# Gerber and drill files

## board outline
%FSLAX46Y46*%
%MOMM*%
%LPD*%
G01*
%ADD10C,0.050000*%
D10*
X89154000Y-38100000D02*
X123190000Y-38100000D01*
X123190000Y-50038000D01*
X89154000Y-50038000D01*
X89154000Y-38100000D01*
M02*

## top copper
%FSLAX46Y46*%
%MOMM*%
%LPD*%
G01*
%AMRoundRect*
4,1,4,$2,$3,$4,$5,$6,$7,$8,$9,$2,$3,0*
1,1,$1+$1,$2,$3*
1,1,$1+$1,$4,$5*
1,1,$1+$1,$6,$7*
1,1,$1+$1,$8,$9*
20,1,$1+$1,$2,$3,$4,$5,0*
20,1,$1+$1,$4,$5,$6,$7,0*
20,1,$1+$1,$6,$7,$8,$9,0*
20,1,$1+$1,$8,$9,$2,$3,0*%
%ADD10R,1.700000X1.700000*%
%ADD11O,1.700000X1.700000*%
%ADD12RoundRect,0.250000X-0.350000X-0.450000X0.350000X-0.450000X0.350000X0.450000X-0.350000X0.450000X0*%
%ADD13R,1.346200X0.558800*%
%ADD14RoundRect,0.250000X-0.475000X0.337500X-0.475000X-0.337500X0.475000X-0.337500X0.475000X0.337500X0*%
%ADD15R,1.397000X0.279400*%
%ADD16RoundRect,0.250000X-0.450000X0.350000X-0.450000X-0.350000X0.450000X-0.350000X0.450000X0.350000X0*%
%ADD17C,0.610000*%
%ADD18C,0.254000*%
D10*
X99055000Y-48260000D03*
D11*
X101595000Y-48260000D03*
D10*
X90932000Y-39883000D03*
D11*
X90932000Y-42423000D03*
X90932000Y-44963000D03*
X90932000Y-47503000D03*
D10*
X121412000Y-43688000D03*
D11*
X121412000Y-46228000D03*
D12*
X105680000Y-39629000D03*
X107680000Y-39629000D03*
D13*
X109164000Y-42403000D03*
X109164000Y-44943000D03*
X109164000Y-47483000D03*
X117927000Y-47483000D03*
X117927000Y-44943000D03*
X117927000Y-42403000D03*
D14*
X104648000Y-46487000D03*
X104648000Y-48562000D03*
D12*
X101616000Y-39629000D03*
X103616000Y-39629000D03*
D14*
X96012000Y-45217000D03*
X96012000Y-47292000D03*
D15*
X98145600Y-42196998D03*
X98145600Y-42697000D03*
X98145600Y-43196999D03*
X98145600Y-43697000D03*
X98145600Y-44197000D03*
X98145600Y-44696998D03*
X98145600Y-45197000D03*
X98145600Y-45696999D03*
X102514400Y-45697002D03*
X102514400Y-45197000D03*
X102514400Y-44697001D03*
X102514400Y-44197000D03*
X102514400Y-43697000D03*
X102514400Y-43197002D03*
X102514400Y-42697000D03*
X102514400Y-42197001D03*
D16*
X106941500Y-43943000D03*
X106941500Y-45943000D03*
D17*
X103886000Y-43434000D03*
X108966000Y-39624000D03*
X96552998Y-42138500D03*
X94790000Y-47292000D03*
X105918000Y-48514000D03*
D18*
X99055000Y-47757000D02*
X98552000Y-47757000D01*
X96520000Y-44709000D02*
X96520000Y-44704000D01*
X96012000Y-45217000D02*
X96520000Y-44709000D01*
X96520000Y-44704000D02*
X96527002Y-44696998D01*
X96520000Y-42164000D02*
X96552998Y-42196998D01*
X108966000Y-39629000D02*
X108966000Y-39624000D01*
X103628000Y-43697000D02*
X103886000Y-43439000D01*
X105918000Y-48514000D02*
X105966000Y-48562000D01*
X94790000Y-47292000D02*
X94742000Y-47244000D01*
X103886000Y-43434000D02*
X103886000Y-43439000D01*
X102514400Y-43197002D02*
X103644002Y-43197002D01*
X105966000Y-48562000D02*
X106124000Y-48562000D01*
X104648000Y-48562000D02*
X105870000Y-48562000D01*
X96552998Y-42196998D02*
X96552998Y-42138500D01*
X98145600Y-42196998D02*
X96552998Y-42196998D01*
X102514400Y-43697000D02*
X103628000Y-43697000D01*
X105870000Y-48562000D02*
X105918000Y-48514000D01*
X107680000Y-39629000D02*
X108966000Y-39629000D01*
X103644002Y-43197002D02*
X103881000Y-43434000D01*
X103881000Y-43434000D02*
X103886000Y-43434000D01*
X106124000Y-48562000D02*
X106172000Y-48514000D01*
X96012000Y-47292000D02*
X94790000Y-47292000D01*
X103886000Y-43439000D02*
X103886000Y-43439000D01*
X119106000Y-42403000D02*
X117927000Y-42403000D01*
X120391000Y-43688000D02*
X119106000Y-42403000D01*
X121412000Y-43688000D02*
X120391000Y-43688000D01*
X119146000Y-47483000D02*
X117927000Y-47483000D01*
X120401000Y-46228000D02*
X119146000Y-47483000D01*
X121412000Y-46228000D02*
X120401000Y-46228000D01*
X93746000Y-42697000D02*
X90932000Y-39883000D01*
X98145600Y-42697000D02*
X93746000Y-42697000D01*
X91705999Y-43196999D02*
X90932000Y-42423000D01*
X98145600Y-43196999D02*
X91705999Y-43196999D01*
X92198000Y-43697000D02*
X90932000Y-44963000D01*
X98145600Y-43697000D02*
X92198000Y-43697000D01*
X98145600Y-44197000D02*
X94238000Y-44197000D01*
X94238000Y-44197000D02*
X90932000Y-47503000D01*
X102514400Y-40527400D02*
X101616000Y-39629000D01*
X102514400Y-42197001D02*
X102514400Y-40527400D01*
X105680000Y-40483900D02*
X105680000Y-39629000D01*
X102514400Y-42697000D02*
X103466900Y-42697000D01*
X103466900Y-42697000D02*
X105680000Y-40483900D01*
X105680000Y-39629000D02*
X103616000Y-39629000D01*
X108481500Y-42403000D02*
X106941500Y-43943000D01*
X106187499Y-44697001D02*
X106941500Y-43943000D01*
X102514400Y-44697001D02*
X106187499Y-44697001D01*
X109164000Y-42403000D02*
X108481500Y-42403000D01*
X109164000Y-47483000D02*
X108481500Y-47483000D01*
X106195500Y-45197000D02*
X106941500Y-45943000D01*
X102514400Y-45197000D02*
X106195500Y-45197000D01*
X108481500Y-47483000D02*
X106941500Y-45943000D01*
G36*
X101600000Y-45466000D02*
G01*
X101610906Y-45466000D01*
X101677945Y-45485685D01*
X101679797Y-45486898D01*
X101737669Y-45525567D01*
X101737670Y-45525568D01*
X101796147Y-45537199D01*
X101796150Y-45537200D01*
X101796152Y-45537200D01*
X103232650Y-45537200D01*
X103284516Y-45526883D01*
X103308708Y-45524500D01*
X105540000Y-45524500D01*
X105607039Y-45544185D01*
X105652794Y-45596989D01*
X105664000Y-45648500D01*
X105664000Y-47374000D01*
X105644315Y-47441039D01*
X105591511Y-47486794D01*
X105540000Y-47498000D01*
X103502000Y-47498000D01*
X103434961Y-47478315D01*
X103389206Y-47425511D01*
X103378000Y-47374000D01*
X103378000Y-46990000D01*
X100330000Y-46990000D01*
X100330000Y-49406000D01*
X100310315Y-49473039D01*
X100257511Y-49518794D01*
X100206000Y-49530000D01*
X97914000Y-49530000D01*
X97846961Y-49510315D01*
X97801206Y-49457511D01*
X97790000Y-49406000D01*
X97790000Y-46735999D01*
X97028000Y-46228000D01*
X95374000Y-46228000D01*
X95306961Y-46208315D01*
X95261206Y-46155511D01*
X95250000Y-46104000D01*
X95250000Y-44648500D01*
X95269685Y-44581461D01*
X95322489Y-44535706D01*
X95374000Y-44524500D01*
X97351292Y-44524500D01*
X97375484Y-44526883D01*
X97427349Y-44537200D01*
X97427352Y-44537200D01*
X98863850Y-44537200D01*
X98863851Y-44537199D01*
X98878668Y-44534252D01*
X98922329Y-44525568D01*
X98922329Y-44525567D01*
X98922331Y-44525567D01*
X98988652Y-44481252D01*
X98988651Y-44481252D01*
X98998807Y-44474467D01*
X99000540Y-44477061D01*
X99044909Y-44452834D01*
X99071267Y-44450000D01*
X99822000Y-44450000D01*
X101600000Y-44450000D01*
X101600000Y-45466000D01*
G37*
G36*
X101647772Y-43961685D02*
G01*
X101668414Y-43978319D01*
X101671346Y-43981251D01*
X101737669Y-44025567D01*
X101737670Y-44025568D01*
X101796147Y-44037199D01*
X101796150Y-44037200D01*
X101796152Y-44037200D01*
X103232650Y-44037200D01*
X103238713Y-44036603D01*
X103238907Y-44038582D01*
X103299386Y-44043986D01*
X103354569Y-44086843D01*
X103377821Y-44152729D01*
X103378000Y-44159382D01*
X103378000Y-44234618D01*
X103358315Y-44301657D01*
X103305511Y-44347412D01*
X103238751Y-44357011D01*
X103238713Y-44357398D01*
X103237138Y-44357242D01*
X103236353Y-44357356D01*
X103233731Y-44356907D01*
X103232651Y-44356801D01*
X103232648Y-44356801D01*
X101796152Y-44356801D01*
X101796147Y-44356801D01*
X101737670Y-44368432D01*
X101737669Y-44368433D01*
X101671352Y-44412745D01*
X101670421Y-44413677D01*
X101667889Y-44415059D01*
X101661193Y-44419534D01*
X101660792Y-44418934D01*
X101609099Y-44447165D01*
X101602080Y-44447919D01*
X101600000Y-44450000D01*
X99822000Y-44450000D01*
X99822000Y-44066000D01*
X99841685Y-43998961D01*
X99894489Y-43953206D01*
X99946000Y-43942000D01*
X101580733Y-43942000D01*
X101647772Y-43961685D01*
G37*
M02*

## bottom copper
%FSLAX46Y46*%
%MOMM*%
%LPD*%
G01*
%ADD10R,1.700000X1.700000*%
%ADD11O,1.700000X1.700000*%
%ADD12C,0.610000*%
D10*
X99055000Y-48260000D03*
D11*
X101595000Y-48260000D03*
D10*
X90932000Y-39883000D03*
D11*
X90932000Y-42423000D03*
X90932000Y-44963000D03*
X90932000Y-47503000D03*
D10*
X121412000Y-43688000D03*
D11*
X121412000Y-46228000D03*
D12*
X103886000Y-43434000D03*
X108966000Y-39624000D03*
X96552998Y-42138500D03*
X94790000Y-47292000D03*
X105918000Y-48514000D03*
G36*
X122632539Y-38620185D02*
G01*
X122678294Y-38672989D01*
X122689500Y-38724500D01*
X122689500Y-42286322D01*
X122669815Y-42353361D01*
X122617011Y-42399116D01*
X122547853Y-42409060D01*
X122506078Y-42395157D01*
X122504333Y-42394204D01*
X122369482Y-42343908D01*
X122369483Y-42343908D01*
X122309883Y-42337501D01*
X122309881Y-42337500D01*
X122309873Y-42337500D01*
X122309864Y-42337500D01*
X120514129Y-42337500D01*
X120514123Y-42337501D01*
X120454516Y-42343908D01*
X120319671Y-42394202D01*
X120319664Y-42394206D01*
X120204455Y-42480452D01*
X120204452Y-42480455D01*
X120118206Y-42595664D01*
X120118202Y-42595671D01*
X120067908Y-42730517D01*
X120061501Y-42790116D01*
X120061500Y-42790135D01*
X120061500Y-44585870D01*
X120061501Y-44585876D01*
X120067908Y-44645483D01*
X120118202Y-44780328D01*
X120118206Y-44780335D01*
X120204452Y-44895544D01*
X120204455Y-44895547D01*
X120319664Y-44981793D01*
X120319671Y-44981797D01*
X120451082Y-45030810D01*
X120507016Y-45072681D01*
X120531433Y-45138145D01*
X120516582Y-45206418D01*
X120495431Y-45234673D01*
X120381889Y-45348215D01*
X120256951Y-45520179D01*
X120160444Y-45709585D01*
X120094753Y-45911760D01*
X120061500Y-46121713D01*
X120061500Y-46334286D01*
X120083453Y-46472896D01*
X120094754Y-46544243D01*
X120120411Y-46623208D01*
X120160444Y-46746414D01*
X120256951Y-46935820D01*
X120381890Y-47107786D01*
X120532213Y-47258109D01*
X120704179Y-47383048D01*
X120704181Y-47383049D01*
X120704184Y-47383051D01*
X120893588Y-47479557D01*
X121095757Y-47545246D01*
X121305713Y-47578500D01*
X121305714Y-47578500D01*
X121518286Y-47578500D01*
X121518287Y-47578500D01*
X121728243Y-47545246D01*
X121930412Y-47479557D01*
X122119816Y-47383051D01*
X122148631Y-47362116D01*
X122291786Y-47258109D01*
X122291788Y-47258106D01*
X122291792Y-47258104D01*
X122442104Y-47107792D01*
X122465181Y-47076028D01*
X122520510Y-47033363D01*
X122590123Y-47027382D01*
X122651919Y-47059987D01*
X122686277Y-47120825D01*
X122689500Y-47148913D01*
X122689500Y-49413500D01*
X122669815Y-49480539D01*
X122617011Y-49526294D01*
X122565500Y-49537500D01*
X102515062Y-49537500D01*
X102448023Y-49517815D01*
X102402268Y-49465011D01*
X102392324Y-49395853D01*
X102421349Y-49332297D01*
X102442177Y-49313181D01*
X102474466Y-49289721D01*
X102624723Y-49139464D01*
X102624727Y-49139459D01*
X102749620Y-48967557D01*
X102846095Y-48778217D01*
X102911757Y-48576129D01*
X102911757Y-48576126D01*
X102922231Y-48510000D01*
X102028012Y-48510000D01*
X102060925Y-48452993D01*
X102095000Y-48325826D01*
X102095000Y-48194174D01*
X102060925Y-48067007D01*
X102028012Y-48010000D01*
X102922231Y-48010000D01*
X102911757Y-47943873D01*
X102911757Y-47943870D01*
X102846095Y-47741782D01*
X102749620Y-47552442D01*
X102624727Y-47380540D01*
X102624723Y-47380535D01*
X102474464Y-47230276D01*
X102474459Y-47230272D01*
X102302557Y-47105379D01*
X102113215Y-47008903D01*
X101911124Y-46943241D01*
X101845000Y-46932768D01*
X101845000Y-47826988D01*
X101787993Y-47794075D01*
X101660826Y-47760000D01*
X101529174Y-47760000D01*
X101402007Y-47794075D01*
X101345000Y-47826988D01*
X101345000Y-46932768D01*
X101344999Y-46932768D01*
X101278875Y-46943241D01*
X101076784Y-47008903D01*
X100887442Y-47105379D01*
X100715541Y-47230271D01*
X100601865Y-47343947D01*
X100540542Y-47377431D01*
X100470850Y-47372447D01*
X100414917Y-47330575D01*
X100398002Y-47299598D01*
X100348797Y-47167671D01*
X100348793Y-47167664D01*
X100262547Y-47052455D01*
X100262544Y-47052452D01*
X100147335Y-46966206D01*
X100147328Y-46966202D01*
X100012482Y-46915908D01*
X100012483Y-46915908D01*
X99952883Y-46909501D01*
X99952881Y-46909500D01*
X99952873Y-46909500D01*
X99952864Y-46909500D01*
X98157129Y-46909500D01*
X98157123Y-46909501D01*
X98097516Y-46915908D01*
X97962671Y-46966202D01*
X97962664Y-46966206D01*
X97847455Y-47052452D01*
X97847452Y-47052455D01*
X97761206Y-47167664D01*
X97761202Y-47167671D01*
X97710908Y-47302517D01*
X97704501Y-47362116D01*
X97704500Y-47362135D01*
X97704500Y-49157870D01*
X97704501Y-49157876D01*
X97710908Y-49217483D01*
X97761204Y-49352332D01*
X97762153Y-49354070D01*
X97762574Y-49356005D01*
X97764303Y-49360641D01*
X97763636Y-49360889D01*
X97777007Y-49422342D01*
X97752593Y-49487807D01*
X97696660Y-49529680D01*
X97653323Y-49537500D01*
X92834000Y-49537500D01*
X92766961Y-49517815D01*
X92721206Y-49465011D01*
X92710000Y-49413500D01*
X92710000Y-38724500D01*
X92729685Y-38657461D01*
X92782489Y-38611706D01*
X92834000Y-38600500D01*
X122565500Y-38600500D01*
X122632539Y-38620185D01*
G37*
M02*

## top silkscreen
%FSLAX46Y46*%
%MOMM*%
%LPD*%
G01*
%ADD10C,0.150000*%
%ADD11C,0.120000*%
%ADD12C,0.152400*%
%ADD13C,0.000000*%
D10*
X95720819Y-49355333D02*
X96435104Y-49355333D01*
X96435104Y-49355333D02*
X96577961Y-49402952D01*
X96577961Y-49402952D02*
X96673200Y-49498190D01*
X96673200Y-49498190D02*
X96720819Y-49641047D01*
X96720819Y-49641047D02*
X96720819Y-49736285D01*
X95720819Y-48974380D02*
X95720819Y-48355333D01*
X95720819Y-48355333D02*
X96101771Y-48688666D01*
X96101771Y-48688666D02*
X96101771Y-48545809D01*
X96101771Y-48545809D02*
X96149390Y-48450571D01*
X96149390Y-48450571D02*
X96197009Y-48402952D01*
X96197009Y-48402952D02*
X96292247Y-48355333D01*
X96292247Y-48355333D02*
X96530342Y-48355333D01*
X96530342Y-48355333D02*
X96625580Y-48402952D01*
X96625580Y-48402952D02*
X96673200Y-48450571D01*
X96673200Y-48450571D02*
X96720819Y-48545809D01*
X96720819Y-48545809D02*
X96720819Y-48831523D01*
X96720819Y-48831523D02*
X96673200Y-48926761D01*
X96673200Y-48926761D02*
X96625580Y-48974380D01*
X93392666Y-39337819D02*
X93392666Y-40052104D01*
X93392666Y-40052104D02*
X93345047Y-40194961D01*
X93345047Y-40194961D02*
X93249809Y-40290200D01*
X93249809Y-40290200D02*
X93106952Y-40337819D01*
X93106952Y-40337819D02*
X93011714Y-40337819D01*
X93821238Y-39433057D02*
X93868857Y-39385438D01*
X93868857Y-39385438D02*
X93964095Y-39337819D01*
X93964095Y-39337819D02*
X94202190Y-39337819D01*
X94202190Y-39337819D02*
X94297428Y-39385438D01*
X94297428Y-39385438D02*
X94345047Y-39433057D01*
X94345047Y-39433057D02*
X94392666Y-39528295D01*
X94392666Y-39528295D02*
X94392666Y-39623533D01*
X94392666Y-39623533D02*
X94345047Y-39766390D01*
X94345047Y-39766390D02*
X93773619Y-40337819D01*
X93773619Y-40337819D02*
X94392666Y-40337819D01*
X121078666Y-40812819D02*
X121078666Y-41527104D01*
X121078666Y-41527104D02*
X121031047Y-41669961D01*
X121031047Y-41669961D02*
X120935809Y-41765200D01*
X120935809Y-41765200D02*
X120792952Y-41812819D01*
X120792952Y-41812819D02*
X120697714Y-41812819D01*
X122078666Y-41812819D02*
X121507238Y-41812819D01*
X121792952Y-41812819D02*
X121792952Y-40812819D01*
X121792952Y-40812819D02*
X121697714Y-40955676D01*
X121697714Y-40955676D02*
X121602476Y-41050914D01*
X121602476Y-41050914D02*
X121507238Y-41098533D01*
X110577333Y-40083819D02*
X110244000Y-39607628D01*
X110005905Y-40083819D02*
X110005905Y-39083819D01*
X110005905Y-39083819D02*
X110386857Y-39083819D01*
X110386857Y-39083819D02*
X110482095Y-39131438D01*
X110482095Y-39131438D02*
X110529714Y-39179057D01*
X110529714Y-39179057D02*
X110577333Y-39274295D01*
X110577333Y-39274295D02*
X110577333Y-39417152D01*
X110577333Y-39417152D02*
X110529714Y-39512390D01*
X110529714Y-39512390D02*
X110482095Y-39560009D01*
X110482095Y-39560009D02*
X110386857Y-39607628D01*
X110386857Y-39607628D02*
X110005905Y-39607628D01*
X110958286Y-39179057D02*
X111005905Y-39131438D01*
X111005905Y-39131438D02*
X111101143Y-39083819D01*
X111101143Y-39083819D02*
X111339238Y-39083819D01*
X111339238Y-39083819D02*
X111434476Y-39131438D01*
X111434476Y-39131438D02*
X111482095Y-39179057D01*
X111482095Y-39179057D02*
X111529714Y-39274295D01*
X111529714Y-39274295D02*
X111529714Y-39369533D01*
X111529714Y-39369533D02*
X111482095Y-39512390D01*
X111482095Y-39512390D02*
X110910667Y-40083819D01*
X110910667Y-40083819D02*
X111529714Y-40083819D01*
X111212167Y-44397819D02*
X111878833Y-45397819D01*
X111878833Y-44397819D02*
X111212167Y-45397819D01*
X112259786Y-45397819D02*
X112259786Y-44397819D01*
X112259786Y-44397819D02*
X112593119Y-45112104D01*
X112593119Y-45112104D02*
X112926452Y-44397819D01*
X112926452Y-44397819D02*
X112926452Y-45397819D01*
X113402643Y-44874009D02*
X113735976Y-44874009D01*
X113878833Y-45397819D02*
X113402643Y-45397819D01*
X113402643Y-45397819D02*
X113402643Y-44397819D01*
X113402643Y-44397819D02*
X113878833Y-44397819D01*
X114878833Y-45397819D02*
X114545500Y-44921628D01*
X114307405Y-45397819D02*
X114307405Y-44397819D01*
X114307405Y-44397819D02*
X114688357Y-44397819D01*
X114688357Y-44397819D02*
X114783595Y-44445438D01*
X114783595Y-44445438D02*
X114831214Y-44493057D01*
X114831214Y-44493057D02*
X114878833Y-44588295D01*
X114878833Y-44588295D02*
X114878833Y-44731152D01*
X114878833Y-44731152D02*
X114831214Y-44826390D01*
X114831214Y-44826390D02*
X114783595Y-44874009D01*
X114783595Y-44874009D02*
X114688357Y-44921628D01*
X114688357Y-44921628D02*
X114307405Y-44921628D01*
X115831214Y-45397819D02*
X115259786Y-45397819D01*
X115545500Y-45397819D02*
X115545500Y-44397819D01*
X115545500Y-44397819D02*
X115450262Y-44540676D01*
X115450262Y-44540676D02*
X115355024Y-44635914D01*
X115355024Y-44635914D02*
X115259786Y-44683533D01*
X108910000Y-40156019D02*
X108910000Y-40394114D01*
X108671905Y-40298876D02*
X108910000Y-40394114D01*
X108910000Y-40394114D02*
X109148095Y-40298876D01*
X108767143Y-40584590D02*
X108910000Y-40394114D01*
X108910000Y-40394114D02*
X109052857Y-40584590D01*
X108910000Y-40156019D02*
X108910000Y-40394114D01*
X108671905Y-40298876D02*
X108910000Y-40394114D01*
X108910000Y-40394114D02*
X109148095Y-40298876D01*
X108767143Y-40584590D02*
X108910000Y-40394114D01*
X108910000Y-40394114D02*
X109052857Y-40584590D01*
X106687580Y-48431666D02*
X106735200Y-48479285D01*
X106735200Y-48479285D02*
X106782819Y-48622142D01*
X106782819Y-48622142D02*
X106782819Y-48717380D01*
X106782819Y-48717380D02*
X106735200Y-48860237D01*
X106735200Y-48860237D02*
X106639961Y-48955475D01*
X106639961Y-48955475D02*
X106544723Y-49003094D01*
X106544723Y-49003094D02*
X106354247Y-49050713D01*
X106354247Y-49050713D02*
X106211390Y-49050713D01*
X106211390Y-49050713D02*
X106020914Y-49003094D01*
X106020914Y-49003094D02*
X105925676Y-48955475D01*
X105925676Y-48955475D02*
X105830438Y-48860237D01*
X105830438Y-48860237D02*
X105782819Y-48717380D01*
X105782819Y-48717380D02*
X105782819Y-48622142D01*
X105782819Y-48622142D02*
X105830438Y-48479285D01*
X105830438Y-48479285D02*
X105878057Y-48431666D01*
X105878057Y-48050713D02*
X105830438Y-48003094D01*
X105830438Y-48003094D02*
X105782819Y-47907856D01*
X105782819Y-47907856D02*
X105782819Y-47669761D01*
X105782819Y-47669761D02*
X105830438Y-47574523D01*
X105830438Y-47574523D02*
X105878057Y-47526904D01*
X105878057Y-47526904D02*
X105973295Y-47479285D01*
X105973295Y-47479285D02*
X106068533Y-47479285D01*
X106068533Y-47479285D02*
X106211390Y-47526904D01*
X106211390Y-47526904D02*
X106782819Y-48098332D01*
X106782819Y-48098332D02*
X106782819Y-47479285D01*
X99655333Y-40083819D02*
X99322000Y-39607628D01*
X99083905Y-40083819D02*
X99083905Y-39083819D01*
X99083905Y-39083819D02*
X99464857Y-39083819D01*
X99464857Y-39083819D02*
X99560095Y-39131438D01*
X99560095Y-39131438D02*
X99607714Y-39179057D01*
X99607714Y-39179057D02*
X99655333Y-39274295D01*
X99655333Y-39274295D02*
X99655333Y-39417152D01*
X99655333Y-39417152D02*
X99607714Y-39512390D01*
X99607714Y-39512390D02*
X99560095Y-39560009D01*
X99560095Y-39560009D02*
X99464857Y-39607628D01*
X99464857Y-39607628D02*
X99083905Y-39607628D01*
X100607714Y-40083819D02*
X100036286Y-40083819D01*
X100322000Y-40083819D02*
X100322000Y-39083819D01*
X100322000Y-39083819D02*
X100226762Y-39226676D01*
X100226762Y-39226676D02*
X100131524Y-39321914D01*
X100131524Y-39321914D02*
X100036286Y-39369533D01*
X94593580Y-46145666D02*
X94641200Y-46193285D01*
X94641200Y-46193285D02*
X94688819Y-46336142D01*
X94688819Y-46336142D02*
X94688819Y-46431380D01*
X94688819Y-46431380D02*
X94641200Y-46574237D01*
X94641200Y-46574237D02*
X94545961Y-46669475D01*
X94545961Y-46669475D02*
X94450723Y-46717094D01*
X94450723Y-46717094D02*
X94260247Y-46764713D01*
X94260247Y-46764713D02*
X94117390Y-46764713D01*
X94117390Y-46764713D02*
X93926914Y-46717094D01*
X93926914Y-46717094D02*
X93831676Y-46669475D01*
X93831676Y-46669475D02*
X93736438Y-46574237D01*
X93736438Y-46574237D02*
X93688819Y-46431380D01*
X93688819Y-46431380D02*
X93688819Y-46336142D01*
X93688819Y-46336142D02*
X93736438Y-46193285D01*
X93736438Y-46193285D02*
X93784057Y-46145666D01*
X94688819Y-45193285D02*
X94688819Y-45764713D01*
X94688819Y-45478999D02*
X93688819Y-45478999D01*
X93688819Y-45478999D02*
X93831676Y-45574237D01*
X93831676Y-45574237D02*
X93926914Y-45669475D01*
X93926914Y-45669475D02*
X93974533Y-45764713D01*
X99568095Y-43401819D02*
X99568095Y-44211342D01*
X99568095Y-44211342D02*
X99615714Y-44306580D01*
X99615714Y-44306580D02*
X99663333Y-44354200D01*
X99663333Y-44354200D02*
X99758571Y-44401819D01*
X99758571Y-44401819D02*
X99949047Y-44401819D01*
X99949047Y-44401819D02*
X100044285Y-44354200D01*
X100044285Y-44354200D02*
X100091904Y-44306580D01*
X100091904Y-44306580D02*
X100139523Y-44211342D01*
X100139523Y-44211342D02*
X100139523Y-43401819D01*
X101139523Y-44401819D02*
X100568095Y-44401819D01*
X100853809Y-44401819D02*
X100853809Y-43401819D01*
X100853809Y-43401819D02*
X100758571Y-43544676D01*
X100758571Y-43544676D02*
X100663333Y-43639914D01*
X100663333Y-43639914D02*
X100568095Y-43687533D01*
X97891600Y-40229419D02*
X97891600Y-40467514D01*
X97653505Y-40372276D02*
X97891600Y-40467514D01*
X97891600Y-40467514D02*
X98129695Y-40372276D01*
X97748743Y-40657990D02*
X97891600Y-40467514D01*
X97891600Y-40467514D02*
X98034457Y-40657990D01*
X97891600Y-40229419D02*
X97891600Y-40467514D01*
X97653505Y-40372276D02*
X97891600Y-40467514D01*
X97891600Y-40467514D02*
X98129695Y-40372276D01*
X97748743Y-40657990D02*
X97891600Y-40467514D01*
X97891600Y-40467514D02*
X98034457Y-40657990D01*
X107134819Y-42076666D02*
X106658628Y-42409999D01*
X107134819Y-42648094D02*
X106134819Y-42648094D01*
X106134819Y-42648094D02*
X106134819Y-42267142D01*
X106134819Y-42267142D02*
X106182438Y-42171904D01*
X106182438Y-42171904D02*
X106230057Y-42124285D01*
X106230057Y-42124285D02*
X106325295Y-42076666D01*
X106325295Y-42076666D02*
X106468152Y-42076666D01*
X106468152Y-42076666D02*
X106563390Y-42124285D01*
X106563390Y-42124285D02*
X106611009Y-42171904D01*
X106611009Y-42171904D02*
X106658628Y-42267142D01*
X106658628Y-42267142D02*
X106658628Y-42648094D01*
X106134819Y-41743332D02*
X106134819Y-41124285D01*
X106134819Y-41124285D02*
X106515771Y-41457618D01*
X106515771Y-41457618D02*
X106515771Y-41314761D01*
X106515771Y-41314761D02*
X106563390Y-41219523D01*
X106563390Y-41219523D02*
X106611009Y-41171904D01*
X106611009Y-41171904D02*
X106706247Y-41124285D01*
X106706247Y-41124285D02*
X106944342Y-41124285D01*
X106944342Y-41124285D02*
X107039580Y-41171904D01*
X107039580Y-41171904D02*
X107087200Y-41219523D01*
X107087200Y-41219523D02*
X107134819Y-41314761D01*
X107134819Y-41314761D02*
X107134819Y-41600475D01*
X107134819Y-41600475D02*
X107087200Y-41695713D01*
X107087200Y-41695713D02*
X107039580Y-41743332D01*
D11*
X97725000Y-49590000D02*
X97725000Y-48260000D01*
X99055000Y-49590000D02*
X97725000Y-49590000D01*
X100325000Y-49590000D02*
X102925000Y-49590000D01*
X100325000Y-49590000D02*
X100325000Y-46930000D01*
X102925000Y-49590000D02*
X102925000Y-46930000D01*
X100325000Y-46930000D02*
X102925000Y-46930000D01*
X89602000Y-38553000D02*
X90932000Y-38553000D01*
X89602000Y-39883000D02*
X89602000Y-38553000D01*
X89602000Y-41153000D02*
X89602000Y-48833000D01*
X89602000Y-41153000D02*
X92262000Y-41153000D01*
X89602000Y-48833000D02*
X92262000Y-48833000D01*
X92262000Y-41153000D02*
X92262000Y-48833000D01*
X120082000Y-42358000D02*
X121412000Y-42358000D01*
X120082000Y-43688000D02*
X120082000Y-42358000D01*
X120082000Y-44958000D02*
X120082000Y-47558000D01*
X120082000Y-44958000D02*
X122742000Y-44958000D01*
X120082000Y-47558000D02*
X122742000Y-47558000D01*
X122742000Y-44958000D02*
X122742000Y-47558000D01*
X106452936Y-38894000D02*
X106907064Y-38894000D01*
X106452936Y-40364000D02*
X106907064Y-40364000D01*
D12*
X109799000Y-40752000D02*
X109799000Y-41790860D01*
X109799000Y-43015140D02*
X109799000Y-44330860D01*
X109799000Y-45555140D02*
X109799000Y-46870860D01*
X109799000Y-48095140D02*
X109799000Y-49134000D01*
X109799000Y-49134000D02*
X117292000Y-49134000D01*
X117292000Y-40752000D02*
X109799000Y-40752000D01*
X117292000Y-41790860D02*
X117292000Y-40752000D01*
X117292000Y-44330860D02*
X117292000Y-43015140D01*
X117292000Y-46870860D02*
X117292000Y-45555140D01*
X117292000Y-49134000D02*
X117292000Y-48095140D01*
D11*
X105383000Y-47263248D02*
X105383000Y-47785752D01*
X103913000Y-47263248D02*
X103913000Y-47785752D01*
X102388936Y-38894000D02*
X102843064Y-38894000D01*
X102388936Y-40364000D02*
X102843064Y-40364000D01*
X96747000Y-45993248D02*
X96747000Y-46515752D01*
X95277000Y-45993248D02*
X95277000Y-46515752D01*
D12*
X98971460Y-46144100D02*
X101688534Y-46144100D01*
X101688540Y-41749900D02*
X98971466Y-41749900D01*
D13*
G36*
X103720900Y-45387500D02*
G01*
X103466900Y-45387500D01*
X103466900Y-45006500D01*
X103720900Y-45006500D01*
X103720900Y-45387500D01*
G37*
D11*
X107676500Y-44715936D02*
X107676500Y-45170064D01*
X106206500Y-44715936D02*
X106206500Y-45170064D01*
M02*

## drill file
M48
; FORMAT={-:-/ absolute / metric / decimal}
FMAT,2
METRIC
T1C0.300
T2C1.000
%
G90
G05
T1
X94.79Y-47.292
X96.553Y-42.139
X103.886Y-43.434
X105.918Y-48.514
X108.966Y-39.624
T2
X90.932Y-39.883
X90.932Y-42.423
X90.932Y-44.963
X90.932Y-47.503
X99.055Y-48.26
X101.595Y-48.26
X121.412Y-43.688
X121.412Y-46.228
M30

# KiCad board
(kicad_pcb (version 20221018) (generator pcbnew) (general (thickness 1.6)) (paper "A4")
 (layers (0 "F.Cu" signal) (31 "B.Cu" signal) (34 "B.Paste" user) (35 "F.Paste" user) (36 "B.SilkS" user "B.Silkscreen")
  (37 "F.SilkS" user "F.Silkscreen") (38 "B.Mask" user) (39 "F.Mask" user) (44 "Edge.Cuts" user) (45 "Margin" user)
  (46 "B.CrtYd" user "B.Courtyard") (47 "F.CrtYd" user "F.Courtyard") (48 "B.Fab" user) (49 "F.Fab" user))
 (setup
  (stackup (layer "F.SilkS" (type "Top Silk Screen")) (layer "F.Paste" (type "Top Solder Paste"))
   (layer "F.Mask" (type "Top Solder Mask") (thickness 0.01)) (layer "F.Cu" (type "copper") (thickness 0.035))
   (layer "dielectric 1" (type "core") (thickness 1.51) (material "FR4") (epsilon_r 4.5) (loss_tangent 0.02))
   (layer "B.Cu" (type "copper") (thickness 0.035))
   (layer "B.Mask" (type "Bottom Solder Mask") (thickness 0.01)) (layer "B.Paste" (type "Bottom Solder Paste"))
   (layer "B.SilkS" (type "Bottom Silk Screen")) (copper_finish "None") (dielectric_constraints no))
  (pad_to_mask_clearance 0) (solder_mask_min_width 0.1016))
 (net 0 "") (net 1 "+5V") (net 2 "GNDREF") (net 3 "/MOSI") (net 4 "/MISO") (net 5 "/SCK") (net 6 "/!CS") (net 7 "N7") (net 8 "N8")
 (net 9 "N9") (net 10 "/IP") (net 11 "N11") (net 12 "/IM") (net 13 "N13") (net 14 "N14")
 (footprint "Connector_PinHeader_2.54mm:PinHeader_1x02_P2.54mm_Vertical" (layer "F.Cu") (at 99.055 48.26 90)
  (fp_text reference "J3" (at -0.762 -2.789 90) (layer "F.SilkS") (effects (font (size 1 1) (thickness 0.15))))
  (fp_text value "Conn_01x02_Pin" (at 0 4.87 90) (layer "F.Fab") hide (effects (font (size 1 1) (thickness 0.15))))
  (fp_line (start -1.33 -1.33) (end 0 -1.33) (stroke (width 0.12) (type solid)) (layer "F.SilkS"))
  (fp_line (start -1.33 0) (end -1.33 -1.33) (stroke (width 0.12) (type solid)) (layer "F.SilkS"))
  (fp_line (start -1.33 1.27) (end -1.33 3.87) (stroke (width 0.12) (type solid)) (layer "F.SilkS"))
  (fp_line (start -1.33 1.27) (end 1.33 1.27) (stroke (width 0.12) (type solid)) (layer "F.SilkS"))
  (fp_line (start -1.33 3.87) (end 1.33 3.87) (stroke (width 0.12) (type solid)) (layer "F.SilkS"))
  (fp_line (start 1.33 1.27) (end 1.33 3.87) (stroke (width 0.12) (type solid)) (layer "F.SilkS"))
  (pad "1" thru_hole rect (at 0 0 90) (size 1.7 1.7) (drill 1) (layers "*.Cu" "*.Mask") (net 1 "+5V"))
  (pad "2" thru_hole oval (at 0 2.54 90) (size 1.7 1.7) (drill 1) (layers "*.Cu" "*.Mask") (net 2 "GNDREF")))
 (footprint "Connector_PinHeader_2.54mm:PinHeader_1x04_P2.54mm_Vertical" (layer "F.Cu") (at 90.932 39.883)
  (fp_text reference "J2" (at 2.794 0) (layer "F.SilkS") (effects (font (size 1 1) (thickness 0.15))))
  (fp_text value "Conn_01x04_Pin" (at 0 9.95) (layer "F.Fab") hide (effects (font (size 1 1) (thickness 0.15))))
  (fp_line (start -1.33 -1.33) (end 0 -1.33) (stroke (width 0.12) (type solid)) (layer "F.SilkS"))
  (fp_line (start -1.33 0) (end -1.33 -1.33) (stroke (width 0.12) (type solid)) (layer "F.SilkS"))
  (fp_line (start -1.33 1.27) (end -1.33 8.95) (stroke (width 0.12) (type solid)) (layer "F.SilkS"))
  (fp_line (start -1.33 1.27) (end 1.33 1.27) (stroke (width 0.12) (type solid)) (layer "F.SilkS"))
  (fp_line (start -1.33 8.95) (end 1.33 8.95) (stroke (width 0.12) (type solid)) (layer "F.SilkS"))
  (fp_line (start 1.33 1.27) (end 1.33 8.95) (stroke (width 0.12) (type solid)) (layer "F.SilkS"))
  (pad "1" thru_hole rect (at 0 0) (size 1.7 1.7) (drill 1) (layers "*.Cu" "*.Mask") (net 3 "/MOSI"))
  (pad "2" thru_hole oval (at 0 2.54) (size 1.7 1.7) (drill 1) (layers "*.Cu" "*.Mask") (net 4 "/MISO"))
  (pad "3" thru_hole oval (at 0 5.08) (size 1.7 1.7) (drill 1) (layers "*.Cu" "*.Mask") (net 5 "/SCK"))
  (pad "4" thru_hole oval (at 0 7.62) (size 1.7 1.7) (drill 1) (layers "*.Cu" "*.Mask") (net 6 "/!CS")))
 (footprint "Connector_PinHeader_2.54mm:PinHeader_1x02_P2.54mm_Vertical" (layer "F.Cu") (at 121.412 43.688)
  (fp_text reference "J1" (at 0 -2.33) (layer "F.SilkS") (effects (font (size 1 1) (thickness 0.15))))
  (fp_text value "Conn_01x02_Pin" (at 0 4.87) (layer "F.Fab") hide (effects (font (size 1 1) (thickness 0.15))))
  (fp_line (start -1.33 -1.33) (end 0 -1.33) (stroke (width 0.12) (type solid)) (layer "F.SilkS"))
  (fp_line (start -1.33 0) (end -1.33 -1.33) (stroke (width 0.12) (type solid)) (layer "F.SilkS"))
  (fp_line (start -1.33 1.27) (end -1.33 3.87) (stroke (width 0.12) (type solid)) (layer "F.SilkS"))
  (fp_line (start -1.33 1.27) (end 1.33 1.27) (stroke (width 0.12) (type solid)) (layer "F.SilkS"))
  (fp_line (start -1.33 3.87) (end 1.33 3.87) (stroke (width 0.12) (type solid)) (layer "F.SilkS"))
  (fp_line (start 1.33 1.27) (end 1.33 3.87) (stroke (width 0.12) (type solid)) (layer "F.SilkS"))
  (pad "1" thru_hole rect (at 0 0) (size 1.7 1.7) (drill 1) (layers "*.Cu" "*.Mask") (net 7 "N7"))
  (pad "2" thru_hole oval (at 0 2.54) (size 1.7 1.7) (drill 1) (layers "*.Cu" "*.Mask") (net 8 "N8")))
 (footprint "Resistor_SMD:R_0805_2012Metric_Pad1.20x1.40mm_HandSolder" (layer "F.Cu") (at 106.68 39.629)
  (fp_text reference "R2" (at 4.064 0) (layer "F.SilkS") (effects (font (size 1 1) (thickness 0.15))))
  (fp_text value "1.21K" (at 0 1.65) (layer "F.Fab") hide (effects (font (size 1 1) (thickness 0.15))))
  (fp_line (start -0.227064 -0.735) (end 0.227064 -0.735) (stroke (width 0.12) (type solid)) (layer "F.SilkS"))
  (fp_line (start -0.227064 0.735) (end 0.227064 0.735) (stroke (width 0.12) (type solid)) (layer "F.SilkS"))
  (pad "1" smd roundrect (at -1 0) (size 1.2 1.4) (layers "F.Cu" "F.Paste" "F.Mask") (roundrect_rratio 0.2083333333) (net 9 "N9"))
  (pad "2" smd roundrect (at 1 0) (size 1.2 1.4) (layers "F.Cu" "F.Paste" "F.Mask") (roundrect_rratio 0.2083333333) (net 2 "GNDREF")))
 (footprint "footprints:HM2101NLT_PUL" (layer "F.Cu") (at 113.5455 44.943)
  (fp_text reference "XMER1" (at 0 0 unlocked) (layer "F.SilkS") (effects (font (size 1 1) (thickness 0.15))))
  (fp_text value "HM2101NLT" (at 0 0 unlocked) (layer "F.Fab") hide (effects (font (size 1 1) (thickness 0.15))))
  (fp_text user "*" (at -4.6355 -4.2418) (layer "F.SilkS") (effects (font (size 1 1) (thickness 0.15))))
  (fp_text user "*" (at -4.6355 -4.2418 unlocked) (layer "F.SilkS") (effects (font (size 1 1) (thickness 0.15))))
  (fp_line (start -3.7465 -4.191) (end -3.7465 -3.15214) (stroke (width 0.1524) (type solid)) (layer "F.SilkS"))
  (fp_line (start -3.7465 -1.92786) (end -3.7465 -0.61214) (stroke (width 0.1524) (type solid)) (layer "F.SilkS"))
  (fp_line (start -3.7465 0.61214) (end -3.7465 1.92786) (stroke (width 0.1524) (type solid)) (layer "F.SilkS"))
  (fp_line (start -3.7465 3.15214) (end -3.7465 4.191) (stroke (width 0.1524) (type solid)) (layer "F.SilkS"))
  (fp_line (start -3.7465 4.191) (end 3.7465 4.191) (stroke (width 0.1524) (type solid)) (layer "F.SilkS"))
  (fp_line (start 3.7465 -4.191) (end -3.7465 -4.191) (stroke (width 0.1524) (type solid)) (layer "F.SilkS"))
  (fp_line (start 3.7465 -3.15214) (end 3.7465 -4.191) (stroke (width 0.1524) (type solid)) (layer "F.SilkS"))
  (fp_line (start 3.7465 -0.61214) (end 3.7465 -1.92786) (stroke (width 0.1524) (type solid)) (layer "F.SilkS"))
  (fp_line (start 3.7465 1.92786) (end 3.7465 0.61214) (stroke (width 0.1524) (type solid)) (layer "F.SilkS"))
  (fp_line (start 3.7465 4.191) (end 3.7465 3.15214) (stroke (width 0.1524) (type solid)) (layer "F.SilkS"))
  (pad "1" smd rect (at -4.3815 -2.54) (size 1.3462 0.5588) (layers "F.Cu" "F.Paste" "F.Mask") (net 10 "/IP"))
  (pad "2" smd rect (at -4.3815 0) (size 1.3462 0.5588) (layers "F.Cu" "F.Paste" "F.Mask") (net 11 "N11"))
  (pad "3" smd rect (at -4.3815 2.54) (size 1.3462 0.5588) (layers "F.Cu" "F.Paste" "F.Mask") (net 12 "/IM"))
  (pad "4" smd rect (at 4.3815 2.54) (size 1.3462 0.5588) (layers "F.Cu" "F.Paste" "F.Mask") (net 8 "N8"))
  (pad "5" smd rect (at 4.3815 0) (size 1.3462 0.5588) (layers "F.Cu" "F.Paste" "F.Mask") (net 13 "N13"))
  (pad "6" smd rect (at 4.3815 -2.54) (size 1.3462 0.5588) (layers "F.Cu" "F.Paste" "F.Mask") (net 7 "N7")))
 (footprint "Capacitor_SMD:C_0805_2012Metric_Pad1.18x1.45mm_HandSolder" (layer "F.Cu") (at 104.648 47.5245 -90)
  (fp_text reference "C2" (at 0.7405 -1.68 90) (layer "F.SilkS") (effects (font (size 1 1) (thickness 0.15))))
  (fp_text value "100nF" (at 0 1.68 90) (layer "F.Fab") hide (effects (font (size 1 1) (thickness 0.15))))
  (fp_line (start -0.261252 -0.735) (end 0.261252 -0.735) (stroke (width 0.12) (type solid)) (layer "F.SilkS"))
  (fp_line (start -0.261252 0.735) (end 0.261252 0.735) (stroke (width 0.12) (type solid)) (layer "F.SilkS"))
  (pad "1" smd roundrect (at -1.0375 0 270) (size 1.175 1.45) (layers "F.Cu" "F.Paste" "F.Mask") (roundrect_rratio 0.2127659574)
   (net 1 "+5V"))
  (pad "2" smd roundrect (at 1.0375 0 270) (size 1.175 1.45) (layers "F.Cu" "F.Paste" "F.Mask") (roundrect_rratio 0.2127659574)
   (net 2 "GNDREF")))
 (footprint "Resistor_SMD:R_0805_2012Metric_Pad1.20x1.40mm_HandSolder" (layer "F.Cu") (at 102.616 39.629)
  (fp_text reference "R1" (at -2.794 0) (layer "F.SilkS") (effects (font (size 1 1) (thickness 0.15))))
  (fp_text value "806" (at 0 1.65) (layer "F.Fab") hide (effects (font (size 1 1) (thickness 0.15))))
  (fp_line (start -0.227064 -0.735) (end 0.227064 -0.735) (stroke (width 0.12) (type solid)) (layer "F.SilkS"))
  (fp_line (start -0.227064 0.735) (end 0.227064 0.735) (stroke (width 0.12) (type solid)) (layer "F.SilkS"))
  (pad "1" smd roundrect (at -1 0) (size 1.2 1.4) (layers "F.Cu" "F.Paste" "F.Mask") (roundrect_rratio 0.2083333333) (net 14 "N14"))
  (pad "2" smd roundrect (at 1 0) (size 1.2 1.4) (layers "F.Cu" "F.Paste" "F.Mask") (roundrect_rratio 0.2083333333) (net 9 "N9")))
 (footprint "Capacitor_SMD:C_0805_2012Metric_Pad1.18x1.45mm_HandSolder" (layer "F.Cu") (at 96.012 46.2545 -90)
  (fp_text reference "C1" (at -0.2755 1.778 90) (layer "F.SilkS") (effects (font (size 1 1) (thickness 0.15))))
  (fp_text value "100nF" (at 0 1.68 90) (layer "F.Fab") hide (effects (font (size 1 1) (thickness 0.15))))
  (fp_line (start -0.261252 -0.735) (end 0.261252 -0.735) (stroke (width 0.12) (type solid)) (layer "F.SilkS"))
  (fp_line (start -0.261252 0.735) (end 0.261252 0.735) (stroke (width 0.12) (type solid)) (layer "F.SilkS"))
  (pad "1" smd roundrect (at -1.0375 0 270) (size 1.175 1.45) (layers "F.Cu" "F.Paste" "F.Mask") (roundrect_rratio 0.2127659574)
   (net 1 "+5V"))
  (pad "2" smd roundrect (at 1.0375 0 270) (size 1.175 1.45) (layers "F.Cu" "F.Paste" "F.Mask") (roundrect_rratio 0.2127659574)
   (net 2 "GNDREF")))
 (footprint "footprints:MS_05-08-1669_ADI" (layer "F.Cu") (at 100.33 43.947)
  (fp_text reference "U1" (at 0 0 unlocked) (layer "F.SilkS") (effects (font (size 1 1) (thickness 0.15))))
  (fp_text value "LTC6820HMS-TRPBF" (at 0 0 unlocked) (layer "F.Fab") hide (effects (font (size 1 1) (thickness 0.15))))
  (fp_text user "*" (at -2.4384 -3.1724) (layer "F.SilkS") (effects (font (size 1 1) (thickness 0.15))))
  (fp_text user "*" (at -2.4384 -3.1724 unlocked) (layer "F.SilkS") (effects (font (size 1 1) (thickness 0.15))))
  (fp_line (start -1.35854 2.1971) (end 1.358534 2.1971) (stroke (width 0.1524) (type solid)) (layer "F.SilkS"))
  (fp_line (start 1.35854 -2.1971) (end -1.358534 -2.1971) (stroke (width 0.1524) (type solid)) (layer "F.SilkS"))
  (fp_poly
   (pts (xy 3.3909 1.0595) (xy 3.3909 1.4405) (xy 3.1369 1.4405) (xy 3.1369 1.0595)) (stroke (width 0) (type solid)) (fill solid)
   (layer "F.SilkS"))
  (pad "1" smd rect (at -2.1844 -1.750002) (size 1.397 0.2794) (layers "F.Cu" "F.Paste" "F.Mask") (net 2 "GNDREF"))
  (pad "2" smd rect (at -2.1844 -1.25) (size 1.397 0.2794) (layers "F.Cu" "F.Paste" "F.Mask") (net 3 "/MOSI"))
  (pad "3" smd rect (at -2.1844 -0.750001) (size 1.397 0.2794) (layers "F.Cu" "F.Paste" "F.Mask") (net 4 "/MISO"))
  (pad "4" smd rect (at -2.1844 -0.25) (size 1.397 0.2794) (layers "F.Cu" "F.Paste" "F.Mask") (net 5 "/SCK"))
  (pad "5" smd rect (at -2.1844 0.25) (size 1.397 0.2794) (layers "F.Cu" "F.Paste" "F.Mask") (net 6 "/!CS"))
  (pad "6" smd rect (at -2.1844 0.749998) (size 1.397 0.2794) (layers "F.Cu" "F.Paste" "F.Mask") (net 1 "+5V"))
  (pad "7" smd rect (at -2.1844 1.25) (size 1.397 0.2794) (layers "F.Cu" "F.Paste" "F.Mask") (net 1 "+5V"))
  (pad "8" smd rect (at -2.1844 1.749999) (size 1.397 0.2794) (layers "F.Cu" "F.Paste" "F.Mask") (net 1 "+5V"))
  (pad "9" smd rect (at 2.1844 1.750002) (size 1.397 0.2794) (layers "F.Cu" "F.Paste" "F.Mask") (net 1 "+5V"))
  (pad "10" smd rect (at 2.1844 1.25) (size 1.397 0.2794) (layers "F.Cu" "F.Paste" "F.Mask") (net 12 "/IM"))
  (pad "11" smd rect (at 2.1844 0.750001) (size 1.397 0.2794) (layers "F.Cu" "F.Paste" "F.Mask") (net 10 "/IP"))
  (pad "12" smd rect (at 2.1844 0.25) (size 1.397 0.2794) (layers "F.Cu" "F.Paste" "F.Mask") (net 1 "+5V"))
  (pad "13" smd rect (at 2.1844 -0.25) (size 1.397 0.2794) (layers "F.Cu" "F.Paste" "F.Mask") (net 2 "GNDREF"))
  (pad "14" smd rect (at 2.1844 -0.749998) (size 1.397 0.2794) (layers "F.Cu" "F.Paste" "F.Mask") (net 2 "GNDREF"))
  (pad "15" smd rect (at 2.1844 -1.25) (size 1.397 0.2794) (layers "F.Cu" "F.Paste" "F.Mask") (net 9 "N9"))
  (pad "16" smd rect (at 2.1844 -1.749999) (size 1.397 0.2794) (layers "F.Cu" "F.Paste" "F.Mask") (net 14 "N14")))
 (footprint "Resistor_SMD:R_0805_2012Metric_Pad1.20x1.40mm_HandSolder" (layer "F.Cu") (at 106.9415 44.943 -90)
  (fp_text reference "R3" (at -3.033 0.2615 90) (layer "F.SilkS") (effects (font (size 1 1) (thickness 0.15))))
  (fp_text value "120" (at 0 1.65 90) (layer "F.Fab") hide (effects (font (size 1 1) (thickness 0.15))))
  (fp_line (start -0.227064 -0.735) (end 0.227064 -0.735) (stroke (width 0.12) (type solid)) (layer "F.SilkS"))
  (fp_line (start -0.227064 0.735) (end 0.227064 0.735) (stroke (width 0.12) (type solid)) (layer "F.SilkS"))
  (pad "1" smd roundrect (at -1 0 270) (size 1.2 1.4) (layers "F.Cu" "F.Paste" "F.Mask") (roundrect_rratio 0.2083333333) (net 10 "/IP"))
  (pad "2" smd roundrect (at 1 0 270) (size 1.2 1.4) (layers "F.Cu" "F.Paste" "F.Mask") (roundrect_rratio 0.2083333333) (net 12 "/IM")))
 (gr_rect (start 89.154 38.1) (end 123.19 50.038) (stroke (width 0.05) (type default)) (fill none) (layer "Edge.Cuts"))
 (segment (start 99.055 47.757) (end 98.552 47.757) (width 0.254) (layer "F.Cu") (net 1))
 (segment (start 96.52 44.709) (end 96.52 44.704) (width 0.254) (layer "F.Cu") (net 1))
 (segment (start 96.012 45.217) (end 96.52 44.709) (width 0.254) (layer "F.Cu") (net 1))
 (segment (start 96.52 44.704) (end 96.527002 44.696998) (width 0.254) (layer "F.Cu") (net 1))
 (segment (start 96.52 42.164) (end 96.552998 42.196998) (width 0.254) (layer "F.Cu") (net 2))
 (segment (start 108.966 39.629) (end 108.966 39.624) (width 0.254) (layer "F.Cu") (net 2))
 (segment (start 103.628 43.697) (end 103.886 43.439) (width 0.254) (layer "F.Cu") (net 2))
 (segment (start 105.918 48.514) (end 105.966 48.562) (width 0.254) (layer "F.Cu") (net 2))
 (segment (start 94.79 47.292) (end 94.742 47.244) (width 0.254) (layer "F.Cu") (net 2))
 (segment (start 103.886 43.434) (end 103.886 43.439) (width 0.254) (layer "F.Cu") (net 2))
 (segment (start 102.5144 43.197002) (end 103.644002 43.197002) (width 0.254) (layer "F.Cu") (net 2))
 (segment (start 105.966 48.562) (end 106.124 48.562) (width 0.254) (layer "F.Cu") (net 2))
 (segment (start 104.648 48.562) (end 105.87 48.562) (width 0.254) (layer "F.Cu") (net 2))
 (segment (start 96.552998 42.196998) (end 96.552998 42.1385) (width 0.254) (layer "F.Cu") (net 2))
 (segment (start 98.1456 42.196998) (end 96.552998 42.196998) (width 0.254) (layer "F.Cu") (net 2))
 (segment (start 102.5144 43.697) (end 103.628 43.697) (width 0.254) (layer "F.Cu") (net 2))
 (segment (start 105.87 48.562) (end 105.918 48.514) (width 0.254) (layer "F.Cu") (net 2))
 (segment (start 107.68 39.629) (end 108.966 39.629) (width 0.254) (layer "F.Cu") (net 2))
 (segment (start 103.644002 43.197002) (end 103.881 43.434) (width 0.254) (layer "F.Cu") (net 2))
 (segment (start 103.881 43.434) (end 103.886 43.434) (width 0.254) (layer "F.Cu") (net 2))
 (segment (start 106.124 48.562) (end 106.172 48.514) (width 0.254) (layer "F.Cu") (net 2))
 (segment (start 96.012 47.292) (end 94.79 47.292) (width 0.254) (layer "F.Cu") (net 2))
 (segment (start 103.886 43.439) (end 103.886 43.439) (width 0.254) (layer "F.Cu") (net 2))
 (via (at 103.886 43.434) (size 0.61) (drill 0.3) (layers "F.Cu" "B.Cu") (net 2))
 (via (at 108.966 39.624) (size 0.61) (drill 0.3) (layers "F.Cu" "B.Cu") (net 2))
 (via (at 96.552998 42.1385) (size 0.61) (drill 0.3) (layers "F.Cu" "B.Cu") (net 2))
 (via (at 94.79 47.292) (size 0.61) (drill 0.3) (layers "F.Cu" "B.Cu") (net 2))
 (via (at 105.918 48.514) (size 0.61) (drill 0.3) (layers "F.Cu" "B.Cu") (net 2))
 (segment (start 119.106 42.403) (end 117.927 42.403) (width 0.254) (layer "F.Cu") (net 7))
 (segment (start 120.391 43.688) (end 119.106 42.403) (width 0.254) (layer "F.Cu") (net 7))
 (segment (start 121.412 43.688) (end 120.391 43.688) (width 0.254) (layer "F.Cu") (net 7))
 (segment (start 119.146 47.483) (end 117.927 47.483) (width 0.254) (layer "F.Cu") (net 8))
 (segment (start 120.401 46.228) (end 119.146 47.483) (width 0.254) (layer "F.Cu") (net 8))
 (segment (start 121.412 46.228) (end 120.401 46.228) (width 0.254) (layer "F.Cu") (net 8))
 (segment (start 93.746 42.697) (end 90.932 39.883) (width 0.254) (layer "F.Cu") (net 3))
 (segment (start 98.1456 42.697) (end 93.746 42.697) (width 0.254) (layer "F.Cu") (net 3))
 (segment (start 91.705999 43.196999) (end 90.932 42.423) (width 0.254) (layer "F.Cu") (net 4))
 (segment (start 98.1456 43.196999) (end 91.705999 43.196999) (width 0.254) (layer "F.Cu") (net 4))
 (segment (start 92.198 43.697) (end 90.932 44.963) (width 0.254) (layer "F.Cu") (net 5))
 (segment (start 98.1456 43.697) (end 92.198 43.697) (width 0.254) (layer "F.Cu") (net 5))
 (segment (start 98.1456 44.197) (end 94.238 44.197) (width 0.254) (layer "F.Cu") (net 6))
 (segment (start 94.238 44.197) (end 90.932 47.503) (width 0.254) (layer "F.Cu") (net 6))
 (segment (start 102.5144 40.5274) (end 101.616 39.629) (width 0.254) (layer "F.Cu") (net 14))
 (segment (start 102.5144 42.197001) (end 102.5144 40.5274) (width 0.254) (layer "F.Cu") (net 14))
 (segment (start 105.68 40.4839) (end 105.68 39.629) (width 0.254) (layer "F.Cu") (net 9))
 (segment (start 102.5144 42.697) (end 103.4669 42.697) (width 0.254) (layer "F.Cu") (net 9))
 (segment (start 103.4669 42.697) (end 105.68 40.4839) (width 0.254) (layer "F.Cu") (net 9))
 (segment (start 105.68 39.629) (end 103.616 39.629) (width 0.254) (layer "F.Cu") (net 9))
 (segment (start 108.4815 42.403) (end 106.9415 43.943) (width 0.254) (layer "F.Cu") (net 10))
 (segment (start 106.187499 44.697001) (end 106.9415 43.943) (width 0.254) (layer "F.Cu") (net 10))
 (segment (start 102.5144 44.697001) (end 106.187499 44.697001) (width 0.254) (layer "F.Cu") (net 10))
 (segment (start 109.164 42.403) (end 108.4815 42.403) (width 0.254) (layer "F.Cu") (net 10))
 (segment (start 109.164 47.483) (end 108.4815 47.483) (width 0.254) (layer "F.Cu") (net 12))
 (segment (start 106.1955 45.197) (end 106.9415 45.943) (width 0.254) (layer "F.Cu") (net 12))
 (segment (start 102.5144 45.197) (end 106.1955 45.197) (width 0.254) (layer "F.Cu") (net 12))
 (segment (start 108.4815 47.483) (end 106.9415 45.943) (width 0.254) (layer "F.Cu") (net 12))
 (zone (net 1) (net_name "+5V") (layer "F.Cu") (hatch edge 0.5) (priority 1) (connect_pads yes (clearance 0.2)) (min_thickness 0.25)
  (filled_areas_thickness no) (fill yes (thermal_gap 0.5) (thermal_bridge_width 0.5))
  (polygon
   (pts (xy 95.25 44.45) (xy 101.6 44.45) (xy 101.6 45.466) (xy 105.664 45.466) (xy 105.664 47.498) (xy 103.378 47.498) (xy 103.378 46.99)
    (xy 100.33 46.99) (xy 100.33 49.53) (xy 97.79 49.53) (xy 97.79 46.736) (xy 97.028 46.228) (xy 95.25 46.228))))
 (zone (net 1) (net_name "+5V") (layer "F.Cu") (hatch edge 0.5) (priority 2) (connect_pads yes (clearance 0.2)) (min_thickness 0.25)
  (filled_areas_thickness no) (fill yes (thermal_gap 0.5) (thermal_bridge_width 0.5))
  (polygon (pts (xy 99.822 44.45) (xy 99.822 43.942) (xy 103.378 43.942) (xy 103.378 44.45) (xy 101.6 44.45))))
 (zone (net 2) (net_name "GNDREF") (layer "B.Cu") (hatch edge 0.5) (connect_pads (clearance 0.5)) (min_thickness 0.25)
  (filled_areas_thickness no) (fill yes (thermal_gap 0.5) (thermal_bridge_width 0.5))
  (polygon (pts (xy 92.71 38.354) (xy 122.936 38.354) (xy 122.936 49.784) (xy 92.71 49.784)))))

